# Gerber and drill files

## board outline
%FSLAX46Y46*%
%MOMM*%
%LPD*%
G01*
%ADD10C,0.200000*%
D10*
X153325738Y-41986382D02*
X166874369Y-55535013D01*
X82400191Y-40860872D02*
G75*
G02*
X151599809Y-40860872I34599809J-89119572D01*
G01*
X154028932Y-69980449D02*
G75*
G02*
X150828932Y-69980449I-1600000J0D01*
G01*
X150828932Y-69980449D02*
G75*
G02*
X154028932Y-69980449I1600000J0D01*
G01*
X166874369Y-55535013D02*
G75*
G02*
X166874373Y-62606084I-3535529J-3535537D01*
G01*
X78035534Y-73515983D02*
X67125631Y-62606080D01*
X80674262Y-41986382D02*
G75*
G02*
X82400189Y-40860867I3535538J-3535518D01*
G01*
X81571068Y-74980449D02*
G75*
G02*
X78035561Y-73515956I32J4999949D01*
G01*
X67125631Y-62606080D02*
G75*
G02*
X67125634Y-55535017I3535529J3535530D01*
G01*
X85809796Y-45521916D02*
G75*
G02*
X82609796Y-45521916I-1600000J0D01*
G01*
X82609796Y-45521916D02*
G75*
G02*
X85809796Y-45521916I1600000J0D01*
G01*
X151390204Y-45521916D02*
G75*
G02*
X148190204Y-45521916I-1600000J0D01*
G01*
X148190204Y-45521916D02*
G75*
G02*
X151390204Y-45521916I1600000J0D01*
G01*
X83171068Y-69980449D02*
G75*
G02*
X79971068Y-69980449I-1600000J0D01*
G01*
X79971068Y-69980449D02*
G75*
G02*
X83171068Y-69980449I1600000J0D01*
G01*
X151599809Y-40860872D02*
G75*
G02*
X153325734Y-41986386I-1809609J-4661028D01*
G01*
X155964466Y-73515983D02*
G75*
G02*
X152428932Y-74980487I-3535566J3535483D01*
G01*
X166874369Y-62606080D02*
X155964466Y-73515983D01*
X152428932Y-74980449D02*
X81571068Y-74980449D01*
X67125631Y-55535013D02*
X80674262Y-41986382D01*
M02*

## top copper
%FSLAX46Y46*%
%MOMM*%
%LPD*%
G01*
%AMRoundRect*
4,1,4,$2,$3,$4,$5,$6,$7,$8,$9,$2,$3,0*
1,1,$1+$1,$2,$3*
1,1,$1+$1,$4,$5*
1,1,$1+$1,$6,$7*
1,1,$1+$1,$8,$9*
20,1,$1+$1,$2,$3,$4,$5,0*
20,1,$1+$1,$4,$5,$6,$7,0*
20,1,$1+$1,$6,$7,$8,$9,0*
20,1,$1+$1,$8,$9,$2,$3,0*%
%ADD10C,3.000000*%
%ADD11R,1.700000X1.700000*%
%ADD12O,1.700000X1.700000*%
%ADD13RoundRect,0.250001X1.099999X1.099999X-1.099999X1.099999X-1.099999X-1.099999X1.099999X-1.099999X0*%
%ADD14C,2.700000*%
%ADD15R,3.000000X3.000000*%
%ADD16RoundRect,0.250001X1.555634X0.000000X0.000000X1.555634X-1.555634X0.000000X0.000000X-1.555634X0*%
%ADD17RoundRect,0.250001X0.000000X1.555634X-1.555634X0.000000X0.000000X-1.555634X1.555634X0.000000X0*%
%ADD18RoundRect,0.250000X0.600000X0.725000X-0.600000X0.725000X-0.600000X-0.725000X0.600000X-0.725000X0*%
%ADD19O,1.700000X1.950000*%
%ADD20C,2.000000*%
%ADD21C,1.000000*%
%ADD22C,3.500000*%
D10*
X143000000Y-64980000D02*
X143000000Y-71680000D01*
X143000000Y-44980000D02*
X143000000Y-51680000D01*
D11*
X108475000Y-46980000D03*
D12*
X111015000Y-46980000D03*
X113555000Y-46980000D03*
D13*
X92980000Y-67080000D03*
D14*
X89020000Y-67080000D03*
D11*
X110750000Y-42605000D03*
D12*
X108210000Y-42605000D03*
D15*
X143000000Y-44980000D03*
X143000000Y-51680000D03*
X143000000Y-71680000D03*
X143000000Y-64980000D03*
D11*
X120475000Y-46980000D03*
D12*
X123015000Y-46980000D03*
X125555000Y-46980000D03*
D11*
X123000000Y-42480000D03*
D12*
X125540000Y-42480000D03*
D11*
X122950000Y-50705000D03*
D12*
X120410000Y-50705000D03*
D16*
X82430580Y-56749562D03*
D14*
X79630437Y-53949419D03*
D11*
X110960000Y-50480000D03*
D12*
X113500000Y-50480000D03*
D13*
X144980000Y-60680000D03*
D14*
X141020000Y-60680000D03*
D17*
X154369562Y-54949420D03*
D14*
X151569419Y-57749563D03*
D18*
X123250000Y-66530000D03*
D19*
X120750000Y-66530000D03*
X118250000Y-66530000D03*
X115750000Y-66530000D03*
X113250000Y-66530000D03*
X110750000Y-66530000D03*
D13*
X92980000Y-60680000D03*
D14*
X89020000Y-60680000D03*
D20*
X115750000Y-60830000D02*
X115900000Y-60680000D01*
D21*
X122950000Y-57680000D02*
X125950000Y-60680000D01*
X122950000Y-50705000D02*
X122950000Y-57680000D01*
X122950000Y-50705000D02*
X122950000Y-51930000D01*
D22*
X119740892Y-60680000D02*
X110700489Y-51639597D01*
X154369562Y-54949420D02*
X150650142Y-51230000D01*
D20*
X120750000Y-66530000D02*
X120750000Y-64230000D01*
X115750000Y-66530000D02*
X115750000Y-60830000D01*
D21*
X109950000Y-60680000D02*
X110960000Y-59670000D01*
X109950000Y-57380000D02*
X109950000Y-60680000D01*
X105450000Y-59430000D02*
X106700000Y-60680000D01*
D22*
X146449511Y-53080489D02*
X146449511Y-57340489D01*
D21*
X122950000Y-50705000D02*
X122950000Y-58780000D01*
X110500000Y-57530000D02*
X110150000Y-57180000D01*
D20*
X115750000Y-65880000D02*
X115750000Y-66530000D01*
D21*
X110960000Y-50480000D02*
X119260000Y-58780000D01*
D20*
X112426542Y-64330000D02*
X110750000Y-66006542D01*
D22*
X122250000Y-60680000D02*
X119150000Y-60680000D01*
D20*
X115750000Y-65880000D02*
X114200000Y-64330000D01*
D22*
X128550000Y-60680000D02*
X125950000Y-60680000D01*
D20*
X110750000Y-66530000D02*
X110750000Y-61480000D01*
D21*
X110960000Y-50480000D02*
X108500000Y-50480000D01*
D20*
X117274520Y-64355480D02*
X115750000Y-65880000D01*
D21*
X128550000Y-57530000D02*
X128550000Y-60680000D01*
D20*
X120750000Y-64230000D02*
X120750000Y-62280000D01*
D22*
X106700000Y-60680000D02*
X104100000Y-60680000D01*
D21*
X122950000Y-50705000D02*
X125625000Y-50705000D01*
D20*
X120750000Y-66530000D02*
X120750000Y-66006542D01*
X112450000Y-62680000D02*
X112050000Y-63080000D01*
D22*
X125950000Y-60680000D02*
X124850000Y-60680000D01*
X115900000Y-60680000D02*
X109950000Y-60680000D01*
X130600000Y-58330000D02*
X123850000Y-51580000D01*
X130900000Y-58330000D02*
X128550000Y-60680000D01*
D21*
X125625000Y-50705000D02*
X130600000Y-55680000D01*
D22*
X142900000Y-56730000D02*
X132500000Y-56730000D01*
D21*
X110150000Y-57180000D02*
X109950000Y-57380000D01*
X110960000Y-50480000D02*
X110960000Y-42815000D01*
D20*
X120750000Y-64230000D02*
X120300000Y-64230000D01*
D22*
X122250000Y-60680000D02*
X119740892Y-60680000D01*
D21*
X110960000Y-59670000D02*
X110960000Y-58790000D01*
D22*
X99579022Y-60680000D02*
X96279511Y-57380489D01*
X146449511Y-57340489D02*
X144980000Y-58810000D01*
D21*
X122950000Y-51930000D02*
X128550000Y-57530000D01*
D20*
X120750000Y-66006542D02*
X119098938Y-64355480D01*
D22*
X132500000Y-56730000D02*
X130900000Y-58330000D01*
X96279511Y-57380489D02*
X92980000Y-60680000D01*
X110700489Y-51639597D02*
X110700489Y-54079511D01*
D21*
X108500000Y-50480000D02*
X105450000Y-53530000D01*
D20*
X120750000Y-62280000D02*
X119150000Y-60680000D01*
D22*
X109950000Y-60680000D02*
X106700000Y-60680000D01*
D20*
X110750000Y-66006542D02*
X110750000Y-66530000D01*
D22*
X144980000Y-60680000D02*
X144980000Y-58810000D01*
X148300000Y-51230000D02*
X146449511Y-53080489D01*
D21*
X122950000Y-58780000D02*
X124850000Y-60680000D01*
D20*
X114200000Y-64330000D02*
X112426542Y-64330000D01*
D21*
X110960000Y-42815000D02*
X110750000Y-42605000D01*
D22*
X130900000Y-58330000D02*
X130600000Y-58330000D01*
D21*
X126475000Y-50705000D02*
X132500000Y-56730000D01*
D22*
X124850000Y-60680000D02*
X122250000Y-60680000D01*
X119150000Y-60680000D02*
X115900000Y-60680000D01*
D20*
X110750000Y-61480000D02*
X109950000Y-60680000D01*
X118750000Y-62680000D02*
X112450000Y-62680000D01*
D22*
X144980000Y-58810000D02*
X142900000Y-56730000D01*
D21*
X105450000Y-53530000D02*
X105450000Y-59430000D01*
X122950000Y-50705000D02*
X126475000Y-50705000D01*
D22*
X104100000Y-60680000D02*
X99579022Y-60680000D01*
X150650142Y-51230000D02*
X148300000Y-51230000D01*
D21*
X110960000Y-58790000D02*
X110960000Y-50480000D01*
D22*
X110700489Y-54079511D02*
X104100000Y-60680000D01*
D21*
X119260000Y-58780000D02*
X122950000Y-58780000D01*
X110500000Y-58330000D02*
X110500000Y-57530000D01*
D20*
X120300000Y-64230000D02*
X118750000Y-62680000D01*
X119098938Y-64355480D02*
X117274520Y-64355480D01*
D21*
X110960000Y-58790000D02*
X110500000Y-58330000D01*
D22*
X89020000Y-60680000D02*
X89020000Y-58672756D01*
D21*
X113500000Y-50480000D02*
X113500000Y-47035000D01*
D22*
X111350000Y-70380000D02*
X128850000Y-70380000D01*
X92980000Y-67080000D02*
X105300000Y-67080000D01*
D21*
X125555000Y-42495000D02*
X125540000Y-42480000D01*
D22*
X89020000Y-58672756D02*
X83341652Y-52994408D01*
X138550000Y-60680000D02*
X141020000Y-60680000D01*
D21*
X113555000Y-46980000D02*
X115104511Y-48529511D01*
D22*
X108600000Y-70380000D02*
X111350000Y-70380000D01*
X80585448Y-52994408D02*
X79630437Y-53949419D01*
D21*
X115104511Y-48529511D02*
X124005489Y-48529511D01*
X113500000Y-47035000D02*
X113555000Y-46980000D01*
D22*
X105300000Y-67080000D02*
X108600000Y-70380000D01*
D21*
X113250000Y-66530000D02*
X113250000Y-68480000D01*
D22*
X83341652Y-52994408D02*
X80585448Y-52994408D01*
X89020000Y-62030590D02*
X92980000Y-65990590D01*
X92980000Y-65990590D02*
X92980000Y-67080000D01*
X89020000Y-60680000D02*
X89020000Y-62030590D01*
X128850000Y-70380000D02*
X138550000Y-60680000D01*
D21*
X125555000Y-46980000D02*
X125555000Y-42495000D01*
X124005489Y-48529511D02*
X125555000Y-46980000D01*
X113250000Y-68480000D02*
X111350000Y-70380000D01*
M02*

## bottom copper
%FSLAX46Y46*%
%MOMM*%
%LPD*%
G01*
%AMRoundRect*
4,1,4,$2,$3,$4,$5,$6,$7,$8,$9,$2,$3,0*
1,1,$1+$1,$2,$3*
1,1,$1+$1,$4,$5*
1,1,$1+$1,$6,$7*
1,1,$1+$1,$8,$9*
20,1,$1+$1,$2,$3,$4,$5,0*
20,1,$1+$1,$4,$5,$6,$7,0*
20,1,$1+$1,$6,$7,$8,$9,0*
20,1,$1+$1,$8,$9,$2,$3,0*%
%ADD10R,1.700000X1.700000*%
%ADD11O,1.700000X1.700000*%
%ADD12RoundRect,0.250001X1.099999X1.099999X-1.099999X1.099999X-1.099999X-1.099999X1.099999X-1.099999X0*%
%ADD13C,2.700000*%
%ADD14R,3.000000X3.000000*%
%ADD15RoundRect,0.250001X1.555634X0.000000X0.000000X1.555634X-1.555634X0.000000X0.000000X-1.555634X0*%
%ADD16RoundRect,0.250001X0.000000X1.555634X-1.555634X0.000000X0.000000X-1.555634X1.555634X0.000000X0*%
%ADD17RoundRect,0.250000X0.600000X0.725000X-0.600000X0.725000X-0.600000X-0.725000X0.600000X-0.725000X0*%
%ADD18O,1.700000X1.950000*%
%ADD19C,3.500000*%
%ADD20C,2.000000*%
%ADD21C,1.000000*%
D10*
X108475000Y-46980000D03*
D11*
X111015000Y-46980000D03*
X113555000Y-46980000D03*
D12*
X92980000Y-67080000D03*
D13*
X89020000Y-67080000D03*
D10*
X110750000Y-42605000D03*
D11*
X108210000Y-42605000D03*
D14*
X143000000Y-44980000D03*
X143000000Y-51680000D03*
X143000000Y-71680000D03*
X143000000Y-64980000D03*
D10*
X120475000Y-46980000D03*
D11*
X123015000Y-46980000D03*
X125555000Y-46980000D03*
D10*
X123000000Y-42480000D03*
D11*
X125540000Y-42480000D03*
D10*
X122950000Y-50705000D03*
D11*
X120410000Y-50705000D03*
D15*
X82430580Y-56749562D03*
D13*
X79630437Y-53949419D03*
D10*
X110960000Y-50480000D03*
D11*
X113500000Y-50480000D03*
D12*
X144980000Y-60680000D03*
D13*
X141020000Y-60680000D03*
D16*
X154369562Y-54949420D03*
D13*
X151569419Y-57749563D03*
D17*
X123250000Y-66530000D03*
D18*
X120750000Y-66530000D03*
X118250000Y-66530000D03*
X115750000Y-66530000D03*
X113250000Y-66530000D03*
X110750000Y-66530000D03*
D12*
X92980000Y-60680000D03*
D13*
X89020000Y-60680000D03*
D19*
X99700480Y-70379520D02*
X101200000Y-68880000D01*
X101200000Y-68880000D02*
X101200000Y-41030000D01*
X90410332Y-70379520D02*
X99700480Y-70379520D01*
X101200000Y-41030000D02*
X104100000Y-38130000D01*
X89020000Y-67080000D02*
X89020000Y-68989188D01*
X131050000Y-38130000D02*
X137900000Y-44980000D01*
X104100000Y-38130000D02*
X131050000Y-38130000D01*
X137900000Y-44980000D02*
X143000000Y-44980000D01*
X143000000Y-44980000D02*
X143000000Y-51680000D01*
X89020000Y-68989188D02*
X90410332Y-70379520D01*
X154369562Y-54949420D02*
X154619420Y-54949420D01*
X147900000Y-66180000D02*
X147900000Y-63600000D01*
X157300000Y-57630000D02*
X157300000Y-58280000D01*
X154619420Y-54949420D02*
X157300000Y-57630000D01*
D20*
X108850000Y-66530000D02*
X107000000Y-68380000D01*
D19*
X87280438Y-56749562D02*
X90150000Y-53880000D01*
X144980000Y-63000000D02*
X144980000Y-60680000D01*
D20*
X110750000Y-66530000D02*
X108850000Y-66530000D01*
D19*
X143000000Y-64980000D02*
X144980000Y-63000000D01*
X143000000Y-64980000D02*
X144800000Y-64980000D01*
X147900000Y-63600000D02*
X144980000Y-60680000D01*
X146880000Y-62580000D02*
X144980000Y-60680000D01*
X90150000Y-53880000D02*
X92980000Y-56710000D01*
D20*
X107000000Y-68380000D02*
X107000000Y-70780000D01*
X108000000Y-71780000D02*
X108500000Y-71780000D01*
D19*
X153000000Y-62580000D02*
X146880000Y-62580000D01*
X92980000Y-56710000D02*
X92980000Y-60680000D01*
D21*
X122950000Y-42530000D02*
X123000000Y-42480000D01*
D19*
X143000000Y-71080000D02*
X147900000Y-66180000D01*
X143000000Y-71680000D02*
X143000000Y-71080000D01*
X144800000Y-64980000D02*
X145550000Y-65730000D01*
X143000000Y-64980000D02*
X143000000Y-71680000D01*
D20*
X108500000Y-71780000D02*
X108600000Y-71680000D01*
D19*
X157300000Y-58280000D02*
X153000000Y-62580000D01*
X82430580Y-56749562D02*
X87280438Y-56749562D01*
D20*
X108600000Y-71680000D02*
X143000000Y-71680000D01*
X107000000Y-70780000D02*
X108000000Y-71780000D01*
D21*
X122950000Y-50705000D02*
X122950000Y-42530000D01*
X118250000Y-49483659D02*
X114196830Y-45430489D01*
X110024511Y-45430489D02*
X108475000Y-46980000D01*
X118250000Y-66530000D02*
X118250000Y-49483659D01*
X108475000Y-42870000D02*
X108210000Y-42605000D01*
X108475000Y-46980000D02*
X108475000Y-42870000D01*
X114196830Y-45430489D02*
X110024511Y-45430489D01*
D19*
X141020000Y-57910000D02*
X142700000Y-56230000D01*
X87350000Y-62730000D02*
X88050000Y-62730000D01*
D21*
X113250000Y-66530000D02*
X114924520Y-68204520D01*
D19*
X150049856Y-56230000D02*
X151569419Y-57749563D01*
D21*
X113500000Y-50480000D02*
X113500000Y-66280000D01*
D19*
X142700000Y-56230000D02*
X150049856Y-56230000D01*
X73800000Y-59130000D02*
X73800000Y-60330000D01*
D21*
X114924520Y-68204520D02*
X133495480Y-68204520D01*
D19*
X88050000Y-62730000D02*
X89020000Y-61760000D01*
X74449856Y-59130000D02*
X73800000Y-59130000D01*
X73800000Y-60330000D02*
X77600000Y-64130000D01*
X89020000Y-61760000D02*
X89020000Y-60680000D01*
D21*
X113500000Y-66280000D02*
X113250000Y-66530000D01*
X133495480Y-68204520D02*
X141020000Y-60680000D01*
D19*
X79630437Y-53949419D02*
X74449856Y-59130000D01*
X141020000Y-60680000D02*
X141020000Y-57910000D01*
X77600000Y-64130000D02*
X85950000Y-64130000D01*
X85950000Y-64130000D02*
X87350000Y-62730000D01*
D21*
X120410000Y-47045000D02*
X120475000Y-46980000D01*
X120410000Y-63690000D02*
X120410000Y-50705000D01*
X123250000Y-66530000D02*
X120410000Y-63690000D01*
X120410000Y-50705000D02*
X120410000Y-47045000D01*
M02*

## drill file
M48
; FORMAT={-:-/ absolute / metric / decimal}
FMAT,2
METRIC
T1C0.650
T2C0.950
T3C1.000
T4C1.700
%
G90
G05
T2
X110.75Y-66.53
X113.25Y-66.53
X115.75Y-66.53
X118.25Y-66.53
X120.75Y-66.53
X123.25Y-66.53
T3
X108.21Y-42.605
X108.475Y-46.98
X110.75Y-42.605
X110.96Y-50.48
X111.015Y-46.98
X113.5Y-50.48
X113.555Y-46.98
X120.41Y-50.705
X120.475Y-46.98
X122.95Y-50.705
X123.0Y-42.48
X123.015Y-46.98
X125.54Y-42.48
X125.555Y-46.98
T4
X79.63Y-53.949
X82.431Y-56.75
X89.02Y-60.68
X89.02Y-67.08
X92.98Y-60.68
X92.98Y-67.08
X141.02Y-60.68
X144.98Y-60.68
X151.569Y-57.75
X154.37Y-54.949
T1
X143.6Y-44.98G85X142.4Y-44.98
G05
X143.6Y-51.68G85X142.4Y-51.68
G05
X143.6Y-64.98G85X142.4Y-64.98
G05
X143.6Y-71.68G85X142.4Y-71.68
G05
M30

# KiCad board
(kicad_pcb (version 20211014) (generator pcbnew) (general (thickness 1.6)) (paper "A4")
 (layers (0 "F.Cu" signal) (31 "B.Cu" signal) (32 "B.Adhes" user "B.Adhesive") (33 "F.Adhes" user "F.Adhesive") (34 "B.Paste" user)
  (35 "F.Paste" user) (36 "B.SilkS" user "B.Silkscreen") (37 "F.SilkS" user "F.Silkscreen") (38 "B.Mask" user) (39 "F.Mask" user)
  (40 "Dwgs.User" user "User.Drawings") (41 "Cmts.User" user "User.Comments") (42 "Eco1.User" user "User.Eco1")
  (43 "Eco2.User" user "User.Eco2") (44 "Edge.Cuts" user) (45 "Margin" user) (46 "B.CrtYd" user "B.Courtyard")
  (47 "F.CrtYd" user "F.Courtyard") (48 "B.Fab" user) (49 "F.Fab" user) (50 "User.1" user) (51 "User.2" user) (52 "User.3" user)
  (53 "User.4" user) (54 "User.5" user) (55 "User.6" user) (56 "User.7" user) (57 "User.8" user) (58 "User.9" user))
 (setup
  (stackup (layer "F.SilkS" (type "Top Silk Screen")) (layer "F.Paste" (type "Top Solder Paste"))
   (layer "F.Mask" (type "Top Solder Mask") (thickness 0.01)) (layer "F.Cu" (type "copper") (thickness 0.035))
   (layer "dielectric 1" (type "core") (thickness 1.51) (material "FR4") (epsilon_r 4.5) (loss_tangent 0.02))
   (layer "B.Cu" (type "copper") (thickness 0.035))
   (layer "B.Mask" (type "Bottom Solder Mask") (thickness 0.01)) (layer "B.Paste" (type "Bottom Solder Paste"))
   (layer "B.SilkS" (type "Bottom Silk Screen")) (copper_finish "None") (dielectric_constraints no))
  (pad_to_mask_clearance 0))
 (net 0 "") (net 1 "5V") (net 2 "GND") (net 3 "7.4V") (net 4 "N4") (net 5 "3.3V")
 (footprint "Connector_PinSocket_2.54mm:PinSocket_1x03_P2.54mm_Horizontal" (layer "F.Cu") (at 108.475 46.98 90)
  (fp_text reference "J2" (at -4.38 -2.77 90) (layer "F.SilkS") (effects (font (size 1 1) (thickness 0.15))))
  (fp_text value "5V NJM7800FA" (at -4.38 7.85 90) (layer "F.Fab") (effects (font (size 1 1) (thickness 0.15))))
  (pad "1" thru_hole rect (at 0 0 90) (size 1.7 1.7) (drill 1) (layers *.Cu *.Mask) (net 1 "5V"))
  (pad "2" thru_hole oval (at 0 2.54 90) (size 1.7 1.7) (drill 1) (layers *.Cu *.Mask) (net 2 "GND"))
  (pad "3" thru_hole oval (at 0 5.08 90) (size 1.7 1.7) (drill 1) (layers *.Cu *.Mask) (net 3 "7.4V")))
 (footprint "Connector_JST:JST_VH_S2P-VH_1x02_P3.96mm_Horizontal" (layer "F.Cu") (at 92.98 67.08 180)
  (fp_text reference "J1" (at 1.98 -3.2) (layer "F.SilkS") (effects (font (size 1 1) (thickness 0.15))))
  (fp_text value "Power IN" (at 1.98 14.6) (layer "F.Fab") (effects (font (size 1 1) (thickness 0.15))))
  (pad "1" thru_hole roundrect (at 0 0 180) (size 2.7 2.7) (drill 1.7) (layers *.Cu *.Mask) (roundrect_rratio 0.09259296296) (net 3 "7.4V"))
  (pad "2" thru_hole circle (at 3.96 0 180) (size 2.7 2.7) (drill 1.7) (layers *.Cu *.Mask) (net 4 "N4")))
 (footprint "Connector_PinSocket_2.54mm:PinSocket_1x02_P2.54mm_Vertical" (layer "F.Cu") (at 110.75 42.605 -90)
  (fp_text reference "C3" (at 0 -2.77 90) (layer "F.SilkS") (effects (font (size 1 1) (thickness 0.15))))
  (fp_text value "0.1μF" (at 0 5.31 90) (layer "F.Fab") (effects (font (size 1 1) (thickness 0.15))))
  (pad "1" thru_hole rect (at 0 0 270) (size 1.7 1.7) (drill 1) (layers *.Cu *.Mask) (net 2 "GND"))
  (pad "2" thru_hole oval (at 0 2.54 270) (size 1.7 1.7) (drill 1) (layers *.Cu *.Mask) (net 1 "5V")))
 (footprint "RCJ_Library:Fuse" (layer "F.Cu") (at 143 58.38 -90)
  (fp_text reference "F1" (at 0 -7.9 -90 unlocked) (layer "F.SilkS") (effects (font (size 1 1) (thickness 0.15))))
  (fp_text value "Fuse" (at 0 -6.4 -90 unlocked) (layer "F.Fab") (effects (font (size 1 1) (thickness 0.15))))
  (fp_line (start 6.6 0) (end 13.3 0) (layer "F.Cu") (width 3))
  (fp_line (start -13.4 0) (end -6.7 0) (layer "F.Cu") (width 3))
  (pad "1" thru_hole rect (at -13.4 0 270) (size 3 3) (drill oval 0.65 1.85) (layers *.Cu *.Mask) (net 4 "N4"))
  (pad "1" thru_hole rect (at -6.7 0 270) (size 3 3) (drill oval 0.65 1.85) (layers *.Cu *.Mask) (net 4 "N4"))
  (pad "2" thru_hole rect (at 13.3 0 270) (size 3 3) (drill oval 0.65 1.85) (layers *.Cu *.Mask) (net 2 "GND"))
  (pad "2" thru_hole rect (at 6.6 0 270) (size 3 3) (drill oval 0.65 1.85) (layers *.Cu *.Mask) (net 2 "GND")))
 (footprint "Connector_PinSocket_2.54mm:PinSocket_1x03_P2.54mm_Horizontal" (layer "F.Cu") (at 120.475 46.98 90)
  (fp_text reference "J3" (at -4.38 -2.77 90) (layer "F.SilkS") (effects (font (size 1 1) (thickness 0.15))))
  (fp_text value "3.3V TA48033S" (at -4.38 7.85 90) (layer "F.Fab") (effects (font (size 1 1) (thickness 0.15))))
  (pad "1" thru_hole rect (at 0 0 90) (size 1.7 1.7) (drill 1) (layers *.Cu *.Mask) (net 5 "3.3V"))
  (pad "2" thru_hole oval (at 0 2.54 90) (size 1.7 1.7) (drill 1) (layers *.Cu *.Mask) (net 2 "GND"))
  (pad "3" thru_hole oval (at 0 5.08 90) (size 1.7 1.7) (drill 1) (layers *.Cu *.Mask) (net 3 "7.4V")))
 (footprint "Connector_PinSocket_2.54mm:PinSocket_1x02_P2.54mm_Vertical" (layer "F.Cu") (at 123 42.48 90)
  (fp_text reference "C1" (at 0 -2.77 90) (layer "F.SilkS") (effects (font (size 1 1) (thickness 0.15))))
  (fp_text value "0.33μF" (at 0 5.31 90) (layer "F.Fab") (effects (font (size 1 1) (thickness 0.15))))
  (pad "1" thru_hole rect (at 0 0 90) (size 1.7 1.7) (drill 1) (layers *.Cu *.Mask) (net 2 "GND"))
  (pad "2" thru_hole oval (at 0 2.54 90) (size 1.7 1.7) (drill 1) (layers *.Cu *.Mask) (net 3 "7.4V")))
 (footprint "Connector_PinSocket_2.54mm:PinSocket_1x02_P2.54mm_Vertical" (layer "B.Cu") (at 122.95 50.705 90)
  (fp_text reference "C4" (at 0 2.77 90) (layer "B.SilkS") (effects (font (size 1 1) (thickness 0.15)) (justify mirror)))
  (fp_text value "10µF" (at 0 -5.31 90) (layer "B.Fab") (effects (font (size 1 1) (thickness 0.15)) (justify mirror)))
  (pad "1" thru_hole rect (at 0 0 90) (size 1.7 1.7) (drill 1) (layers *.Cu *.Mask) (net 2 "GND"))
  (pad "2" thru_hole oval (at 0 -2.54 90) (size 1.7 1.7) (drill 1) (layers *.Cu *.Mask) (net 5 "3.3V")))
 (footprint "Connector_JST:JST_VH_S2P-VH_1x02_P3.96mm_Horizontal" (layer "B.Cu") (at 82.43058 56.749562 135)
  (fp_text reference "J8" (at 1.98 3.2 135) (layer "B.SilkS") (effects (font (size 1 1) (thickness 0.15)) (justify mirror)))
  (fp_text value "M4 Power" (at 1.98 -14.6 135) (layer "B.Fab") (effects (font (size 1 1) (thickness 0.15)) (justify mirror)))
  (pad "1" thru_hole roundrect (at 0 0 135) (size 2.7 2.7) (drill 1.7) (layers *.Cu *.Mask) (roundrect_rratio 0.09259296296) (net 2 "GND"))
  (pad "2" thru_hole circle (at 3.96 0 135) (size 2.7 2.7) (drill 1.7) (layers *.Cu *.Mask) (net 3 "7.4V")))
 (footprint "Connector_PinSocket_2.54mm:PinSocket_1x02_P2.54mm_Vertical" (layer "B.Cu") (at 110.96 50.48 -90)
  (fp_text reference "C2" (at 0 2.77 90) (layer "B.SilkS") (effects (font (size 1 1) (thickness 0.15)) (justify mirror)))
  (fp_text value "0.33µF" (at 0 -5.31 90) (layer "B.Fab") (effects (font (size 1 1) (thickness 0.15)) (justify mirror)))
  (pad "1" thru_hole rect (at 0 0 270) (size 1.7 1.7) (drill 1) (layers *.Cu *.Mask) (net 2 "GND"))
  (pad "2" thru_hole oval (at 0 -2.54 270) (size 1.7 1.7) (drill 1) (layers *.Cu *.Mask) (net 3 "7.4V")))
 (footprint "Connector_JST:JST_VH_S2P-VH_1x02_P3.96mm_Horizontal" (layer "B.Cu") (at 144.98 60.68 180)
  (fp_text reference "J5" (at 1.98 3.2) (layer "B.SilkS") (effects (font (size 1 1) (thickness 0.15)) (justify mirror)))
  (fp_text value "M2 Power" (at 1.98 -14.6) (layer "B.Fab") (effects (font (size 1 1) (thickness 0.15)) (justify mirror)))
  (pad "1" thru_hole roundrect (at 0 0 180) (size 2.7 2.7) (drill 1.7) (layers *.Cu *.Mask) (roundrect_rratio 0.09259296296) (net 2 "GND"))
  (pad "2" thru_hole circle (at 3.96 0 180) (size 2.7 2.7) (drill 1.7) (layers *.Cu *.Mask) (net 3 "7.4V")))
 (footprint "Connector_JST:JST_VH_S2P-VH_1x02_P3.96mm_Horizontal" (layer "B.Cu") (at 154.369562 54.94942 -135)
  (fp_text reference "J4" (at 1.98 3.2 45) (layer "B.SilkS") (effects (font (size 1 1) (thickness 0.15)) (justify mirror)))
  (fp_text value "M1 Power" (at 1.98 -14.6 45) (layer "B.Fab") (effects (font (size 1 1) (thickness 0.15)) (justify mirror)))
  (pad "1" thru_hole roundrect (at 0 0 225) (size 2.7 2.7) (drill 1.7) (layers *.Cu *.Mask) (roundrect_rratio 0.09259296296) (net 2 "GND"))
  (pad "2" thru_hole circle (at 3.96 0 225) (size 2.7 2.7) (drill 1.7) (layers *.Cu *.Mask) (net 3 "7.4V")))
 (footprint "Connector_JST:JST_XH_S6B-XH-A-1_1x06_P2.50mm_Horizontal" (layer "B.Cu") (at 123.25 66.53 180)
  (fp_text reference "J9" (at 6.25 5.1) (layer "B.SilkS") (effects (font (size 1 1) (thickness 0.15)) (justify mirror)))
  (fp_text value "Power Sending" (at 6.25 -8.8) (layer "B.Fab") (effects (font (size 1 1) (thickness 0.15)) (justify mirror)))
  (pad "1" thru_hole roundrect (at 0 0 180) (size 1.7 1.95) (drill 0.95) (layers *.Cu *.Mask) (roundrect_rratio 0.1470588235) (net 5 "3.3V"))
  (pad "2" thru_hole oval (at 2.5 0 180) (size 1.7 1.95) (drill 0.95) (layers *.Cu *.Mask) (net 2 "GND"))
  (pad "3" thru_hole oval (at 5 0 180) (size 1.7 1.95) (drill 0.95) (layers *.Cu *.Mask) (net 1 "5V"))
  (pad "4" thru_hole oval (at 7.5 0 180) (size 1.7 1.95) (drill 0.95) (layers *.Cu *.Mask) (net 2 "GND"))
  (pad "5" thru_hole oval (at 10 0 180) (size 1.7 1.95) (drill 0.95) (layers *.Cu *.Mask) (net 3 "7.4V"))
  (pad "6" thru_hole oval (at 12.5 0 180) (size 1.7 1.95) (drill 0.95) (layers *.Cu *.Mask) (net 2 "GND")))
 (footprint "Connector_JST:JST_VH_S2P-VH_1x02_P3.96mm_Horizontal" (layer "B.Cu") (at 92.98 60.68 180)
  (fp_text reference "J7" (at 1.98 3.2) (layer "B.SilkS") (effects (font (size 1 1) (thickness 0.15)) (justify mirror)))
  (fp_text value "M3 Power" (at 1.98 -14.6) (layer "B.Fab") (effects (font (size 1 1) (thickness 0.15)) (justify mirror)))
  (pad "1" thru_hole roundrect (at 0 0 180) (size 2.7 2.7) (drill 1.7) (layers *.Cu *.Mask) (roundrect_rratio 0.09259296296) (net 2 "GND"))
  (pad "2" thru_hole circle (at 3.96 0 180) (size 2.7 2.7) (drill 1.7) (layers *.Cu *.Mask) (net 3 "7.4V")))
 (gr_line (start 153.325738 41.986382) (end 166.874369 55.535013) (layer "Edge.Cuts") (width 0.2))
 (gr_arc (start 82.400191 40.860872) (mid 117 34.38) (end 151.599809 40.860872) (layer "Edge.Cuts") (width 0.2))
 (gr_circle (center 152.428932 69.980449) (end 150.828932 69.980449) (layer "Edge.Cuts") (width 0.2) (fill none))
 (gr_arc (start 166.874369 55.535013) (mid 168.338835 59.070546) (end 166.874369 62.60608) (layer "Edge.Cuts") (width 0.2))
 (gr_line (start 78.035534 73.515983) (end 67.125631 62.60608) (layer "Edge.Cuts") (width 0.2))
 (gr_arc (start 80.674262 41.986382) (mid 81.47862 41.333757) (end 82.400191 40.860872) (layer "Edge.Cuts") (width 0.2))
 (gr_arc (start 81.571068 74.980449) (mid 79.657651 74.599847) (end 78.035534 73.515983) (layer "Edge.Cuts") (width 0.2))
 (gr_arc (start 67.125631 62.60608) (mid 65.661165 59.070546) (end 67.125631 55.535013) (layer "Edge.Cuts") (width 0.2))
 (gr_circle (center 84.209796 45.521916) (end 82.609796 45.521916) (layer "Edge.Cuts") (width 0.2) (fill none))
 (gr_circle (center 149.790204 45.521916) (end 148.190204 45.521916) (layer "Edge.Cuts") (width 0.2) (fill none))
 (gr_circle (center 81.571068 69.980449) (end 79.971068 69.980449) (layer "Edge.Cuts") (width 0.2) (fill none))
 (gr_arc (start 151.599809 40.860872) (mid 152.52138 41.333757) (end 153.325738 41.986382) (layer "Edge.Cuts") (width 0.2))
 (gr_arc (start 155.964466 73.515983) (mid 154.342349 74.599847) (end 152.428932 74.980449) (layer "Edge.Cuts") (width 0.2))
 (gr_line (start 166.874369 62.60608) (end 155.964466 73.515983) (layer "Edge.Cuts") (width 0.2))
 (gr_line (start 152.428932 74.980449) (end 81.571068 74.980449) (layer "Edge.Cuts") (width 0.2))
 (gr_line (start 67.125631 55.535013) (end 80.674262 41.986382) (layer "Edge.Cuts") (width 0.2))
 (segment (start 99.70048 70.37952) (end 101.2 68.88) (width 3.5) (layer "B.Cu") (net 4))
 (segment (start 101.2 68.88) (end 101.2 41.03) (width 3.5) (layer "B.Cu") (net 4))
 (segment (start 90.410332 70.37952) (end 99.70048 70.37952) (width 3.5) (layer "B.Cu") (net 4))
 (segment (start 101.2 41.03) (end 104.1 38.13) (width 3.5) (layer "B.Cu") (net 4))
 (segment (start 89.02 67.08) (end 89.02 68.989188) (width 3.5) (layer "B.Cu") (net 4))
 (segment (start 131.05 38.13) (end 137.9 44.98) (width 3.5) (layer "B.Cu") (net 4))
 (segment (start 104.1 38.13) (end 131.05 38.13) (width 3.5) (layer "B.Cu") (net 4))
 (segment (start 137.9 44.98) (end 143 44.98) (width 3.5) (layer "B.Cu") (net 4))
 (segment (start 143 44.98) (end 143 51.68) (width 3.5) (layer "B.Cu") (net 4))
 (segment (start 89.02 68.989188) (end 90.410332 70.37952) (width 3.5) (layer "B.Cu") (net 4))
 (segment (start 115.75 60.83) (end 115.9 60.68) (width 2) (layer "F.Cu") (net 2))
 (segment (start 122.95 57.68) (end 125.95 60.68) (width 1) (layer "F.Cu") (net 2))
 (segment (start 122.95 50.705) (end 122.95 57.68) (width 1) (layer "F.Cu") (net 2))
 (segment (start 122.95 50.705) (end 122.95 51.93) (width 1) (layer "F.Cu") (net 2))
 (segment (start 119.740892 60.68) (end 110.700489 51.639597) (width 3.5) (layer "F.Cu") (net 2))
 (segment (start 154.369562 54.94942) (end 150.650142 51.23) (width 3.5) (layer "F.Cu") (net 2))
 (segment (start 120.75 66.53) (end 120.75 64.23) (width 2) (layer "F.Cu") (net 2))
 (segment (start 115.75 66.53) (end 115.75 60.83) (width 2) (layer "F.Cu") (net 2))
 (segment (start 109.95 60.68) (end 110.96 59.67) (width 1) (layer "F.Cu") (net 2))
 (segment (start 109.95 57.38) (end 109.95 60.68) (width 1) (layer "F.Cu") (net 2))
 (segment (start 105.45 59.43) (end 106.7 60.68) (width 1) (layer "F.Cu") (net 2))
 (segment (start 146.449511 53.080489) (end 146.449511 57.340489) (width 3.5) (layer "F.Cu") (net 2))
 (segment (start 122.95 50.705) (end 122.95 58.78) (width 1) (layer "F.Cu") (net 2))
 (segment (start 110.5 57.53) (end 110.15 57.18) (width 1) (layer "F.Cu") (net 2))
 (segment (start 115.75 65.88) (end 115.75 66.53) (width 2) (layer "F.Cu") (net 2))
 (segment (start 110.96 50.48) (end 119.26 58.78) (width 1) (layer "F.Cu") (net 2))
 (segment (start 112.426542 64.33) (end 110.75 66.006542) (width 2) (layer "F.Cu") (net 2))
 (segment (start 122.25 60.68) (end 119.15 60.68) (width 3.5) (layer "F.Cu") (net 2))
 (segment (start 115.75 65.88) (end 114.2 64.33) (width 2) (layer "F.Cu") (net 2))
 (segment (start 128.55 60.68) (end 125.95 60.68) (width 3.5) (layer "F.Cu") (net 2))
 (segment (start 110.75 66.53) (end 110.75 61.48) (width 2) (layer "F.Cu") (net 2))
 (segment (start 110.96 50.48) (end 108.5 50.48) (width 1) (layer "F.Cu") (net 2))
 (segment (start 117.27452 64.35548) (end 115.75 65.88) (width 2) (layer "F.Cu") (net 2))
 (segment (start 128.55 57.53) (end 128.55 60.68) (width 1) (layer "F.Cu") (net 2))
 (segment (start 120.75 64.23) (end 120.75 62.28) (width 2) (layer "F.Cu") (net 2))
 (segment (start 106.7 60.68) (end 104.1 60.68) (width 3.5) (layer "F.Cu") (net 2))
 (segment (start 122.95 50.705) (end 125.625 50.705) (width 1) (layer "F.Cu") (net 2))
 (segment (start 120.75 66.53) (end 120.75 66.006542) (width 2) (layer "F.Cu") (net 2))
 (segment (start 112.45 62.68) (end 112.05 63.08) (width 2) (layer "F.Cu") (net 2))
 (segment (start 125.95 60.68) (end 124.85 60.68) (width 3.5) (layer "F.Cu") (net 2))
 (segment (start 115.9 60.68) (end 109.95 60.68) (width 3.5) (layer "F.Cu") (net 2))
 (segment (start 130.6 58.33) (end 123.85 51.58) (width 3.5) (layer "F.Cu") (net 2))
 (segment (start 130.9 58.33) (end 128.55 60.68) (width 3.5) (layer "F.Cu") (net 2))
 (segment (start 125.625 50.705) (end 130.6 55.68) (width 1) (layer "F.Cu") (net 2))
 (segment (start 142.9 56.73) (end 132.5 56.73) (width 3.5) (layer "F.Cu") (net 2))
 (segment (start 110.15 57.18) (end 109.95 57.38) (width 1) (layer "F.Cu") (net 2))
 (segment (start 110.96 50.48) (end 110.96 42.815) (width 1) (layer "F.Cu") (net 2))
 (segment (start 120.75 64.23) (end 120.3 64.23) (width 2) (layer "F.Cu") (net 2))
 (segment (start 122.25 60.68) (end 119.740892 60.68) (width 3.5) (layer "F.Cu") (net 2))
 (segment (start 110.96 59.67) (end 110.96 58.79) (width 1) (layer "F.Cu") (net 2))
 (segment (start 99.579022 60.68) (end 96.279511 57.380489) (width 3.5) (layer "F.Cu") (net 2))
 (segment (start 146.449511 57.340489) (end 144.98 58.81) (width 3.5) (layer "F.Cu") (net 2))
 (segment (start 122.95 51.93) (end 128.55 57.53) (width 1) (layer "F.Cu") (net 2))
 (segment (start 120.75 66.006542) (end 119.098938 64.35548) (width 2) (layer "F.Cu") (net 2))
 (segment (start 132.5 56.73) (end 130.9 58.33) (width 3.5) (layer "F.Cu") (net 2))
 (segment (start 96.279511 57.380489) (end 92.98 60.68) (width 3.5) (layer "F.Cu") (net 2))
 (segment (start 110.700489 51.639597) (end 110.700489 54.079511) (width 3.5) (layer "F.Cu") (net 2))
 (segment (start 108.5 50.48) (end 105.45 53.53) (width 1) (layer "F.Cu") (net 2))
 (segment (start 120.75 62.28) (end 119.15 60.68) (width 2) (layer "F.Cu") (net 2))
 (segment (start 109.95 60.68) (end 106.7 60.68) (width 3.5) (layer "F.Cu") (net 2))
 (segment (start 110.75 66.006542) (end 110.75 66.53) (width 2) (layer "F.Cu") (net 2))
 (segment (start 144.98 60.68) (end 144.98 58.81) (width 3.5) (layer "F.Cu") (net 2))
 (segment (start 148.3 51.23) (end 146.449511 53.080489) (width 3.5) (layer "F.Cu") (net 2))
 (segment (start 122.95 58.78) (end 124.85 60.68) (width 1) (layer "F.Cu") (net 2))
 (segment (start 114.2 64.33) (end 112.426542 64.33) (width 2) (layer "F.Cu") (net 2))
 (segment (start 110.96 42.815) (end 110.75 42.605) (width 1) (layer "F.Cu") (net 2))
 (segment (start 130.9 58.33) (end 130.6 58.33) (width 3.5) (layer "F.Cu") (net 2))
 (segment (start 126.475 50.705) (end 132.5 56.73) (width 1) (layer "F.Cu") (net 2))
 (segment (start 124.85 60.68) (end 122.25 60.68) (width 3.5) (layer "F.Cu") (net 2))
 (segment (start 119.15 60.68) (end 115.9 60.68) (width 3.5) (layer "F.Cu") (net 2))
 (segment (start 110.75 61.48) (end 109.95 60.68) (width 2) (layer "F.Cu") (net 2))
 (segment (start 118.75 62.68) (end 112.45 62.68) (width 2) (layer "F.Cu") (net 2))
 (segment (start 144.98 58.81) (end 142.9 56.73) (width 3.5) (layer "F.Cu") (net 2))
 (segment (start 105.45 53.53) (end 105.45 59.43) (width 1) (layer "F.Cu") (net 2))
 (segment (start 122.95 50.705) (end 126.475 50.705) (width 1) (layer "F.Cu") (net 2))
 (segment (start 104.1 60.68) (end 99.579022 60.68) (width 3.5) (layer "F.Cu") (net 2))
 (segment (start 150.650142 51.23) (end 148.3 51.23) (width 3.5) (layer "F.Cu") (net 2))
 (segment (start 110.96 58.79) (end 110.96 50.48) (width 1) (layer "F.Cu") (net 2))
 (segment (start 110.700489 54.079511) (end 104.1 60.68) (width 3.5) (layer "F.Cu") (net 2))
 (segment (start 119.26 58.78) (end 122.95 58.78) (width 1) (layer "F.Cu") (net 2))
 (segment (start 110.5 58.33) (end 110.5 57.53) (width 1) (layer "F.Cu") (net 2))
 (segment (start 120.3 64.23) (end 118.75 62.68) (width 2) (layer "F.Cu") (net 2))
 (segment (start 119.098938 64.35548) (end 117.27452 64.35548) (width 2) (layer "F.Cu") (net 2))
 (segment (start 110.96 58.79) (end 110.5 58.33) (width 1) (layer "F.Cu") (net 2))
 (segment (start 154.369562 54.94942) (end 154.61942 54.94942) (width 3.5) (layer "B.Cu") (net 2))
 (segment (start 147.9 66.18) (end 147.9 63.6) (width 3.5) (layer "B.Cu") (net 2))
 (segment (start 157.3 57.63) (end 157.3 58.28) (width 3.5) (layer "B.Cu") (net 2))
 (segment (start 154.61942 54.94942) (end 157.3 57.63) (width 3.5) (layer "B.Cu") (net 2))
 (segment (start 108.85 66.53) (end 107 68.38) (width 2) (layer "B.Cu") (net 2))
 (segment (start 87.280438 56.749562) (end 90.15 53.88) (width 3.5) (layer "B.Cu") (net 2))
 (segment (start 144.98 63) (end 144.98 60.68) (width 3.5) (layer "B.Cu") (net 2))
 (segment (start 110.75 66.53) (end 108.85 66.53) (width 2) (layer "B.Cu") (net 2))
 (segment (start 143 64.98) (end 144.98 63) (width 3.5) (layer "B.Cu") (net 2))
 (segment (start 143 64.98) (end 144.8 64.98) (width 3.5) (layer "B.Cu") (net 2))
 (segment (start 147.9 63.6) (end 144.98 60.68) (width 3.5) (layer "B.Cu") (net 2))
 (segment (start 146.88 62.58) (end 144.98 60.68) (width 3.5) (layer "B.Cu") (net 2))
 (segment (start 90.15 53.88) (end 92.98 56.71) (width 3.5) (layer "B.Cu") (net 2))
 (segment (start 107 68.38) (end 107 70.78) (width 2) (layer "B.Cu") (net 2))
 (segment (start 108 71.78) (end 108.5 71.78) (width 2) (layer "B.Cu") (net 2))
 (segment (start 153 62.58) (end 146.88 62.58) (width 3.5) (layer "B.Cu") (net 2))
 (segment (start 92.98 56.71) (end 92.98 60.68) (width 3.5) (layer "B.Cu") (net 2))
 (segment (start 122.95 42.53) (end 123 42.48) (width 1) (layer "B.Cu") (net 2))
 (segment (start 143 71.08) (end 147.9 66.18) (width 3.5) (layer "B.Cu") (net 2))
 (segment (start 143 71.68) (end 143 71.08) (width 3.5) (layer "B.Cu") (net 2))
 (segment (start 144.8 64.98) (end 145.55 65.73) (width 3.5) (layer "B.Cu") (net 2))
 (segment (start 143 64.98) (end 143 71.68) (width 3.5) (layer "B.Cu") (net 2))
 (segment (start 108.5 71.78) (end 108.6 71.68) (width 2) (layer "B.Cu") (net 2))
 (segment (start 157.3 58.28) (end 153 62.58) (width 3.5) (layer "B.Cu") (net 2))
 (segment (start 82.43058 56.749562) (end 87.280438 56.749562) (width 3.5) (layer "B.Cu") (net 2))
 (segment (start 108.6 71.68) (end 143 71.68) (width 2) (layer "B.Cu") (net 2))
 (segment (start 107 70.78) (end 108 71.78) (width 2) (layer "B.Cu") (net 2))
 (segment (start 122.95 50.705) (end 122.95 42.53) (width 1) (layer "B.Cu") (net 2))
 (segment (start 118.25 49.483659) (end 114.19683 45.430489) (width 1) (layer "B.Cu") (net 1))
 (segment (start 110.024511 45.430489) (end 108.475 46.98) (width 1) (layer "B.Cu") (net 1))
 (segment (start 118.25 66.53) (end 118.25 49.483659) (width 1) (layer "B.Cu") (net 1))
 (segment (start 108.475 42.87) (end 108.21 42.605) (width 1) (layer "B.Cu") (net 1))
 (segment (start 108.475 46.98) (end 108.475 42.87) (width 1) (layer "B.Cu") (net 1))
 (segment (start 114.19683 45.430489) (end 110.024511 45.430489) (width 1) (layer "B.Cu") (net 1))
 (segment (start 89.02 60.68) (end 89.02 58.672756) (width 3.5) (layer "F.Cu") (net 3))
 (segment (start 113.5 50.48) (end 113.5 47.035) (width 1) (layer "F.Cu") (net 3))
 (segment (start 111.35 70.38) (end 128.85 70.38) (width 3.5) (layer "F.Cu") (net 3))
 (segment (start 92.98 67.08) (end 105.3 67.08) (width 3.5) (layer "F.Cu") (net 3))
 (segment (start 125.555 42.495) (end 125.54 42.48) (width 1) (layer "F.Cu") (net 3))
 (segment (start 89.02 58.672756) (end 83.341652 52.994408) (width 3.5) (layer "F.Cu") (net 3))
 (segment (start 138.55 60.68) (end 141.02 60.68) (width 3.5) (layer "F.Cu") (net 3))
 (segment (start 113.555 46.98) (end 115.104511 48.529511) (width 1) (layer "F.Cu") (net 3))
 (segment (start 108.6 70.38) (end 111.35 70.38) (width 3.5) (layer "F.Cu") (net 3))
 (segment (start 80.585448 52.994408) (end 79.630437 53.949419) (width 3.5) (layer "F.Cu") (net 3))
 (segment (start 115.104511 48.529511) (end 124.005489 48.529511) (width 1) (layer "F.Cu") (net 3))
 (segment (start 113.5 47.035) (end 113.555 46.98) (width 1) (layer "F.Cu") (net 3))
 (segment (start 105.3 67.08) (end 108.6 70.38) (width 3.5) (layer "F.Cu") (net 3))
 (segment (start 113.25 66.53) (end 113.25 68.48) (width 1) (layer "F.Cu") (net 3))
 (segment (start 83.341652 52.994408) (end 80.585448 52.994408) (width 3.5) (layer "F.Cu") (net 3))
 (segment (start 89.02 62.03059) (end 92.98 65.99059) (width 3.5) (layer "F.Cu") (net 3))
 (segment (start 92.98 65.99059) (end 92.98 67.08) (width 3.5) (layer "F.Cu") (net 3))
 (segment (start 89.02 60.68) (end 89.02 62.03059) (width 3.5) (layer "F.Cu") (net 3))
 (segment (start 128.85 70.38) (end 138.55 60.68) (width 3.5) (layer "F.Cu") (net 3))
 (segment (start 125.555 46.98) (end 125.555 42.495) (width 1) (layer "F.Cu") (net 3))
 (segment (start 124.005489 48.529511) (end 125.555 46.98) (width 1) (layer "F.Cu") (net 3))
 (segment (start 113.25 68.48) (end 111.35 70.38) (width 1) (layer "F.Cu") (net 3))
 (segment (start 141.02 57.91) (end 142.7 56.23) (width 3.5) (layer "B.Cu") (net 3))
 (segment (start 87.35 62.73) (end 88.05 62.73) (width 3.5) (layer "B.Cu") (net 3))
 (segment (start 113.25 66.53) (end 114.92452 68.20452) (width 1) (layer "B.Cu") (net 3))
 (segment (start 150.049856 56.23) (end 151.569419 57.749563) (width 3.5) (layer "B.Cu") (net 3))
 (segment (start 113.5 50.48) (end 113.5 66.28) (width 1) (layer "B.Cu") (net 3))
 (segment (start 142.7 56.23) (end 150.049856 56.23) (width 3.5) (layer "B.Cu") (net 3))
 (segment (start 73.8 59.13) (end 73.8 60.33) (width 3.5) (layer "B.Cu") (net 3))
 (segment (start 114.92452 68.20452) (end 133.49548 68.20452) (width 1) (layer "B.Cu") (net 3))
 (segment (start 88.05 62.73) (end 89.02 61.76) (width 3.5) (layer "B.Cu") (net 3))
 (segment (start 74.449856 59.13) (end 73.8 59.13) (width 3.5) (layer "B.Cu") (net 3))
 (segment (start 73.8 60.33) (end 77.6 64.13) (width 3.5) (layer "B.Cu") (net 3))
 (segment (start 89.02 61.76) (end 89.02 60.68) (width 3.5) (layer "B.Cu") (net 3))
 (segment (start 113.5 66.28) (end 113.25 66.53) (width 1) (layer "B.Cu") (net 3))
 (segment (start 133.49548 68.20452) (end 141.02 60.68) (width 1) (layer "B.Cu") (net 3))
 (segment (start 79.630437 53.949419) (end 74.449856 59.13) (width 3.5) (layer "B.Cu") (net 3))
 (segment (start 141.02 60.68) (end 141.02 57.91) (width 3.5) (layer "B.Cu") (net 3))
 (segment (start 77.6 64.13) (end 85.95 64.13) (width 3.5) (layer "B.Cu") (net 3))
 (segment (start 85.95 64.13) (end 87.35 62.73) (width 3.5) (layer "B.Cu") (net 3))
 (segment (start 120.41 47.045) (end 120.475 46.98) (width 1) (layer "B.Cu") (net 5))
 (segment (start 120.41 63.69) (end 120.41 50.705) (width 1) (layer "B.Cu") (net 5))
 (segment (start 123.25 66.53) (end 120.41 63.69) (width 1) (layer "B.Cu") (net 5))
 (segment (start 120.41 50.705) (end 120.41 47.045) (width 1) (layer "B.Cu") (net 5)))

